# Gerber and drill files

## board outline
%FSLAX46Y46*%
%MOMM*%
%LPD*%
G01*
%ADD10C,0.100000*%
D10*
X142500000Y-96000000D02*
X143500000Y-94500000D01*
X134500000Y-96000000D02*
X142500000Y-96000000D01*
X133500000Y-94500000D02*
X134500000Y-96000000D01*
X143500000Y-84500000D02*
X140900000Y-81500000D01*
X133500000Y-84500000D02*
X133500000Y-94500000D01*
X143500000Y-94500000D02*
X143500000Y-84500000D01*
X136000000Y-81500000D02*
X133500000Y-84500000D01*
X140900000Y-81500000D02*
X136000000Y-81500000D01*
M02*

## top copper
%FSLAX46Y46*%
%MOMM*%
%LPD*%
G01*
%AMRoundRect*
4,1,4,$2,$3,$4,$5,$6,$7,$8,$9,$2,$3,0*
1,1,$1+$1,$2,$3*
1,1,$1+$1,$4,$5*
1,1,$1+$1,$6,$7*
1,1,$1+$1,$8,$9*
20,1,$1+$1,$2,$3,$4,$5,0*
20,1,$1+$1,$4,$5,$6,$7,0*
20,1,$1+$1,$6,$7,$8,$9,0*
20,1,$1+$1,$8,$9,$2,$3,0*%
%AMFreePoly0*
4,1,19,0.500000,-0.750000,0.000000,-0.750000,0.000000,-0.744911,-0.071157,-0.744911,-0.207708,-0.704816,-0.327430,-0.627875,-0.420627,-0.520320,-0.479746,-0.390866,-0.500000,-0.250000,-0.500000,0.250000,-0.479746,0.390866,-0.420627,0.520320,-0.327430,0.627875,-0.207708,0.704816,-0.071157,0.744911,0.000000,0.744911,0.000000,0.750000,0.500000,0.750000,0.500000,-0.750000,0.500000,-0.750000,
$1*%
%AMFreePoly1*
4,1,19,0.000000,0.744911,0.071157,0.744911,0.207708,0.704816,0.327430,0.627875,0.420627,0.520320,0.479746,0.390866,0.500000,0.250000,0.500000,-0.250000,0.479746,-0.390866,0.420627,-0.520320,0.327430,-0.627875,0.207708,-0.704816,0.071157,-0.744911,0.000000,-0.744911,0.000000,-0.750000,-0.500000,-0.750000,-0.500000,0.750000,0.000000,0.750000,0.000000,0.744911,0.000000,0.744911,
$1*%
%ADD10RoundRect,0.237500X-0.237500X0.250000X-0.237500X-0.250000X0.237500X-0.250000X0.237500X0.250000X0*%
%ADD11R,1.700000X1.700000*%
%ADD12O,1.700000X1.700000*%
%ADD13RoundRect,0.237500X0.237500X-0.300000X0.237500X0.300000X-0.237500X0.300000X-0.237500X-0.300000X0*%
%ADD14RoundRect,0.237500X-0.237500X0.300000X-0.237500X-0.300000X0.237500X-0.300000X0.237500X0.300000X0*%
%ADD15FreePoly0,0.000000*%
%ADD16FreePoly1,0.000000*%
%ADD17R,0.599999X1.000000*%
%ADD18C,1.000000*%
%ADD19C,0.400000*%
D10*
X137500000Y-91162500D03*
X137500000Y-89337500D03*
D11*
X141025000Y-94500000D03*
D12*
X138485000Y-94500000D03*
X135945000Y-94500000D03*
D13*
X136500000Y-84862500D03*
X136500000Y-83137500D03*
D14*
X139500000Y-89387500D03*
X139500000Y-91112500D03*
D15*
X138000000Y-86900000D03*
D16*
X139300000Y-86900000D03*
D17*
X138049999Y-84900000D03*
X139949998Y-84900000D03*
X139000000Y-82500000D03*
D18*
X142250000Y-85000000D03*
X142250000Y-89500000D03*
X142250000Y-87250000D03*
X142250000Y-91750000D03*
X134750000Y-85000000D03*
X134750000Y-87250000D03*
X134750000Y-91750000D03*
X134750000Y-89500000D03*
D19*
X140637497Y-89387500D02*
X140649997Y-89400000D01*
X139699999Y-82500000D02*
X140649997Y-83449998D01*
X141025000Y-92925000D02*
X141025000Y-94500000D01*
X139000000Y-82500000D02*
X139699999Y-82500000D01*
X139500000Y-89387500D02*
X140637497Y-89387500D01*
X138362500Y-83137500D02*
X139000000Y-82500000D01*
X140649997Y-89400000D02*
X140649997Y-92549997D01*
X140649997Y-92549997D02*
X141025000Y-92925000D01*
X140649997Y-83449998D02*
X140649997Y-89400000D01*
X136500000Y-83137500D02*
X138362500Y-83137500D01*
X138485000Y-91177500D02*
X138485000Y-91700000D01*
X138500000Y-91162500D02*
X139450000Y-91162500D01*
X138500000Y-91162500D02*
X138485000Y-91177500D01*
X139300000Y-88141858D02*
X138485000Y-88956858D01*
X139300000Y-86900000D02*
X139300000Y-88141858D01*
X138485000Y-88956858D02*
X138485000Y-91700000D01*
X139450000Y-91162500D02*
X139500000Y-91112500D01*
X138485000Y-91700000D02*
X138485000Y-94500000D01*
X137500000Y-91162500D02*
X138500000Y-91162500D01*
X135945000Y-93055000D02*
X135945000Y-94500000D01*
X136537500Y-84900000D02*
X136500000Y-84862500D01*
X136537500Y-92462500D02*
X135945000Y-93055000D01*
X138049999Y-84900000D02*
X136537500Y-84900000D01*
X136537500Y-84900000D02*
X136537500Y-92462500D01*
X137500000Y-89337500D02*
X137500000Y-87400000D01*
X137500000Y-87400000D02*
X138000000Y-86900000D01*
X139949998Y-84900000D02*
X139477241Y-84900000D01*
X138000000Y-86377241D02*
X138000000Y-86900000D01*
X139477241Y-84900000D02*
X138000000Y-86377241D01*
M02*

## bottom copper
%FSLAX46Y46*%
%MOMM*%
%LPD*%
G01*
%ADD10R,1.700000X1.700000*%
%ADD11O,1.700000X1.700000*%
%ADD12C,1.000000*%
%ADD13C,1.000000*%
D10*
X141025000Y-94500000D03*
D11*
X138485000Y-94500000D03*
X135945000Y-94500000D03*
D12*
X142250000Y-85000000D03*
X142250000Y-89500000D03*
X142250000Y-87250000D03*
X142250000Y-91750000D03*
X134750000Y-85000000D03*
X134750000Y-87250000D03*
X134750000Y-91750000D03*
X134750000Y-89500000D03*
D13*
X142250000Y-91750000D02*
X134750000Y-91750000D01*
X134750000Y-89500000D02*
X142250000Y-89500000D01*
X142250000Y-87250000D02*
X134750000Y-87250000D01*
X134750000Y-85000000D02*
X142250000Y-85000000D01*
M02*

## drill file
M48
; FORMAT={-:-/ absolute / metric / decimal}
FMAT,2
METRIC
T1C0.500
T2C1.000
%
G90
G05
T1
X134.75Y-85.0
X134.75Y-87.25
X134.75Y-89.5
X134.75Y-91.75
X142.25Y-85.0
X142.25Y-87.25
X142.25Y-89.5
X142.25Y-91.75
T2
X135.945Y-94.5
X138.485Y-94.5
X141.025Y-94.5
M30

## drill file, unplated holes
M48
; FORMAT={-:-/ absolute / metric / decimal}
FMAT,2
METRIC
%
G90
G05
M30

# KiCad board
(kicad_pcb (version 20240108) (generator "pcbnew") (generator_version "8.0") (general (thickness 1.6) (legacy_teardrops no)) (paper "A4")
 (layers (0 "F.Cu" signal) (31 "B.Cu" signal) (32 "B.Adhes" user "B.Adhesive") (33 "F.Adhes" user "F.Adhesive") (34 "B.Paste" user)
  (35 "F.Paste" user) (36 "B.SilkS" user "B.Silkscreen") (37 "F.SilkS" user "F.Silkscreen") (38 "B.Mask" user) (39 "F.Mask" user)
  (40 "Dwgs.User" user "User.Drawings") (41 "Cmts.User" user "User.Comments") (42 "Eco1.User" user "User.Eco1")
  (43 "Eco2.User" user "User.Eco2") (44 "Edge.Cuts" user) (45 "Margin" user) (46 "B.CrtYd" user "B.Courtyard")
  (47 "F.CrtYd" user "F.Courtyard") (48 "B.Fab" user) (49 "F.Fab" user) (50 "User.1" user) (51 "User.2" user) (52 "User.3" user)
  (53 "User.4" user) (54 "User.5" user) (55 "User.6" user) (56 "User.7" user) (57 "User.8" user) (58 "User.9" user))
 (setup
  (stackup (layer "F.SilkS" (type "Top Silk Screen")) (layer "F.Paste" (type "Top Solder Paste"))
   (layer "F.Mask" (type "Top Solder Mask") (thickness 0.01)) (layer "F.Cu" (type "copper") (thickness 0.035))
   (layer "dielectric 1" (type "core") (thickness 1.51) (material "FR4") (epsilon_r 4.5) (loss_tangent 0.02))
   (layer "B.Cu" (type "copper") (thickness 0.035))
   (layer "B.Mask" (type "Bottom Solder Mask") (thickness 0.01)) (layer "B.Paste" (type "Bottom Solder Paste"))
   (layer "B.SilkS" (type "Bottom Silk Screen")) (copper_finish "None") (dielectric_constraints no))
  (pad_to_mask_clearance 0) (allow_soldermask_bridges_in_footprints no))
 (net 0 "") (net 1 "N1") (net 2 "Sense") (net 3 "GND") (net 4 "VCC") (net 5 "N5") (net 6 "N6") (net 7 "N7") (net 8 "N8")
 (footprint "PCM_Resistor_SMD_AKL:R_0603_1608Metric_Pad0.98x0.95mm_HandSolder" (layer "F.Cu") (at 137.5 90.25 -90)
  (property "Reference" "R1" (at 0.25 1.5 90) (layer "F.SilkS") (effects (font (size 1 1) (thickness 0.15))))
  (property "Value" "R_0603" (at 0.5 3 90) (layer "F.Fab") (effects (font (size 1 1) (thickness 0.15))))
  (pad "1" smd roundrect (at -0.9125 0 270) (size 0.975 0.95) (layers "F.Cu" "F.Paste" "F.Mask") (roundrect_rratio 0.25) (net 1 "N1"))
  (pad "2" smd roundrect (at 0.9125 0 270) (size 0.975 0.95) (layers "F.Cu" "F.Paste" "F.Mask") (roundrect_rratio 0.25) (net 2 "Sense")))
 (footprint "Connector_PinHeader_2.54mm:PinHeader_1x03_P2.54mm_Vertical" (layer "F.Cu") (at 141.025 94.5 -90)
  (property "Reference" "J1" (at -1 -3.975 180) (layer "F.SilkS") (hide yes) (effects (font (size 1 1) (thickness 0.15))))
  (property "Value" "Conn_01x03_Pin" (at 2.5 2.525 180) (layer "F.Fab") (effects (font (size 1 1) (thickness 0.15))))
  (pad "1" thru_hole rect (at 0 0 270) (size 1.7 1.7) (drill 1) (layers "*.Cu" "*.Mask") (remove_unused_layers no) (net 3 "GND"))
  (pad "2" thru_hole oval (at 0 2.54 270) (size 1.7 1.7) (drill 1) (layers "*.Cu" "*.Mask") (remove_unused_layers no) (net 2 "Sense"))
  (pad "3" thru_hole oval (at 0 5.08 270) (size 1.7 1.7) (drill 1) (layers "*.Cu" "*.Mask") (remove_unused_layers no) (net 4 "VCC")))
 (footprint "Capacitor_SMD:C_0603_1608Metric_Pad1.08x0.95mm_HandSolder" (layer "F.Cu") (at 136.5 84 90)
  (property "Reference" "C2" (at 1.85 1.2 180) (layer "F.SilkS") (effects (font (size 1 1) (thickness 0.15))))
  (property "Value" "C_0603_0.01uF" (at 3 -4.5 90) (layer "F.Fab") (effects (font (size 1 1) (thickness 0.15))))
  (pad "1" smd roundrect (at -0.8625 0 90) (size 1.075 0.95) (layers "F.Cu" "F.Paste" "F.Mask") (roundrect_rratio 0.25) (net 4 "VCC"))
  (pad "2" smd roundrect (at 0.8625 0 90) (size 1.075 0.95) (layers "F.Cu" "F.Paste" "F.Mask") (roundrect_rratio 0.25) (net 3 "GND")))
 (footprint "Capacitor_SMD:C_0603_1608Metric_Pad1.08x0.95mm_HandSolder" (layer "F.Cu") (at 139.5 90.25 -90)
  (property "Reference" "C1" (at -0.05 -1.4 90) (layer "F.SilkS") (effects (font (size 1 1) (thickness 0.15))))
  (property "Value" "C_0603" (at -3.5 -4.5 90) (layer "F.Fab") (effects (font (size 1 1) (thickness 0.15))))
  (pad "1" smd roundrect (at -0.8625 0 270) (size 1.075 0.95) (layers "F.Cu" "F.Paste" "F.Mask") (roundrect_rratio 0.25) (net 3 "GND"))
  (pad "2" smd roundrect (at 0.8625 0 270) (size 1.075 0.95) (layers "F.Cu" "F.Paste" "F.Mask") (roundrect_rratio 0.25) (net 2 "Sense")))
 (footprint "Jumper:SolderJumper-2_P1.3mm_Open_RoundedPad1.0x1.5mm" (layer "F.Cu") (at 138.65 86.9)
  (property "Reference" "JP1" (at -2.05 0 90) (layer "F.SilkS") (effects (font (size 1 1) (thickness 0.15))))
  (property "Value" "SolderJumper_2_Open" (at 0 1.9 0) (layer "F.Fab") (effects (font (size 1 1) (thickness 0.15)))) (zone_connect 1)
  (pad "1" smd custom (at -0.65 0) (size 1 0.5) (layers "F.Cu" "F.Mask") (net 1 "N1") (zone_connect 2) (thermal_bridge_angle 45)
   (options (clearance outline) (anchor rect)) (primitives))
  (pad "2" smd custom (at 0.65 0) (size 1 0.5) (layers "F.Cu" "F.Mask") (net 2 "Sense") (zone_connect 2) (thermal_bridge_angle 45)
   (options (clearance outline) (anchor rect)) (primitives)))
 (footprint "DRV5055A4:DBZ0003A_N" (layer "F.Cu") (at 139 83.7 90)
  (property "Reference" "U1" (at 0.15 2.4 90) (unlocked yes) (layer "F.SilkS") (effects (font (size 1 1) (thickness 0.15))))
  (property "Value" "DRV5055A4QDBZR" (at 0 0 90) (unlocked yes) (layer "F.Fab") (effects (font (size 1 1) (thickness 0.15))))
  (pad "1" smd rect (at -1.2 -0.950001 180) (size 0.599999 1) (layers "F.Cu" "F.Paste" "F.Mask") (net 4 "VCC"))
  (pad "2" smd rect (at -1.2 0.949998 180) (size 0.599999 1) (layers "F.Cu" "F.Paste" "F.Mask") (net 1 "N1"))
  (pad "3" smd rect (at 1.2 0 180) (size 0.599999 1) (layers "F.Cu" "F.Paste" "F.Mask") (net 3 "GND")))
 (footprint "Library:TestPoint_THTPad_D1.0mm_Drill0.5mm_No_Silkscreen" (layer "B.Cu") (at 142.25 85 90)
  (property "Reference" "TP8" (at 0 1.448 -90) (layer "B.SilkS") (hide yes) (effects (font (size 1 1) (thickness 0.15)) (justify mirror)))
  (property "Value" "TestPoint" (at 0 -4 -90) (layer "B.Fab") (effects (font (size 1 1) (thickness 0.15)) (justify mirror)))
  (pad "1" thru_hole circle (at 0 0 90) (size 1 1) (drill 0.5) (layers "*.Cu" "*.Mask") (remove_unused_layers no) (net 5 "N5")))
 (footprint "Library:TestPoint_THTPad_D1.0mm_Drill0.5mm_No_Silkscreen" (layer "B.Cu") (at 142.25 89.5 90)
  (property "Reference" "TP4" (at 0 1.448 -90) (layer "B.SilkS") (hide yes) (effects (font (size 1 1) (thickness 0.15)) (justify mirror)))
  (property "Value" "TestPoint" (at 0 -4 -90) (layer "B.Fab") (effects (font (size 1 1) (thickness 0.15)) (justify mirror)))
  (pad "1" thru_hole circle (at 0 0 90) (size 1 1) (drill 0.5) (layers "*.Cu" "*.Mask") (remove_unused_layers no) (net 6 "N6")))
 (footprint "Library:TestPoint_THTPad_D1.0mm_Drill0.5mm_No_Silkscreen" (layer "B.Cu") (at 142.25 87.25 90)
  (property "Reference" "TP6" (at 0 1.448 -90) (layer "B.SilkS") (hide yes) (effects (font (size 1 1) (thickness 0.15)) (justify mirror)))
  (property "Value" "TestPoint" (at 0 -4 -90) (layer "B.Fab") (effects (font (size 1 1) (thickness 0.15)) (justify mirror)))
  (pad "1" thru_hole circle (at 0 0 90) (size 1 1) (drill 0.5) (layers "*.Cu" "*.Mask") (remove_unused_layers no) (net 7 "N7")))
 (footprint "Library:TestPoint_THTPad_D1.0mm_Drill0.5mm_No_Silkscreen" (layer "B.Cu") (at 142.25 91.75 90)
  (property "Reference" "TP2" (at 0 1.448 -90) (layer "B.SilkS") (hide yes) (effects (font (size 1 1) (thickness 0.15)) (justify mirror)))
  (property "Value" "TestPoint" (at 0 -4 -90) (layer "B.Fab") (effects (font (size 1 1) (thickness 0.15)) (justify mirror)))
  (pad "1" thru_hole circle (at 0 0 90) (size 1 1) (drill 0.5) (layers "*.Cu" "*.Mask") (remove_unused_layers no) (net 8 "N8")))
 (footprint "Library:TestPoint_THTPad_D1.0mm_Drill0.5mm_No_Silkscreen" (layer "B.Cu") (at 134.75 85 90)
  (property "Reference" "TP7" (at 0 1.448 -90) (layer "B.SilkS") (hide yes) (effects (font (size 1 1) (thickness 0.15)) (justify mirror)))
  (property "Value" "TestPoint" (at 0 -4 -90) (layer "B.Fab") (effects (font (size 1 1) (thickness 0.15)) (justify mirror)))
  (pad "1" thru_hole circle (at 0 0 90) (size 1 1) (drill 0.5) (layers "*.Cu" "*.Mask") (remove_unused_layers no) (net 5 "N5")))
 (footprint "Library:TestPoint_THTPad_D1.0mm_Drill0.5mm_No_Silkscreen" (layer "B.Cu") (at 134.75 87.25 90)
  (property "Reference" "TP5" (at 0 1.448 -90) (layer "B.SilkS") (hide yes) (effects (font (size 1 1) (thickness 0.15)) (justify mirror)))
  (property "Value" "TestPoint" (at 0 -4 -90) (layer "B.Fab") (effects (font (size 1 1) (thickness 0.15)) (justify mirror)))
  (pad "1" thru_hole circle (at 0 0 90) (size 1 1) (drill 0.5) (layers "*.Cu" "*.Mask") (remove_unused_layers no) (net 7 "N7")))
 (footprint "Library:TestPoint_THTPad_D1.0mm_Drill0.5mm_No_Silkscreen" (layer "B.Cu") (at 134.75 91.75 90)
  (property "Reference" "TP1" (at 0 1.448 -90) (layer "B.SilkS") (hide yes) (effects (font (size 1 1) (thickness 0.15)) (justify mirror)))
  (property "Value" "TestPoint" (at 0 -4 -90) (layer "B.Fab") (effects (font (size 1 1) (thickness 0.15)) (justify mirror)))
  (pad "1" thru_hole circle (at 0 0 90) (size 1 1) (drill 0.5) (layers "*.Cu" "*.Mask") (remove_unused_layers no) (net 8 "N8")))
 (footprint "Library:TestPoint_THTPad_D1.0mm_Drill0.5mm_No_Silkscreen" (layer "B.Cu") (at 134.75 89.5 90)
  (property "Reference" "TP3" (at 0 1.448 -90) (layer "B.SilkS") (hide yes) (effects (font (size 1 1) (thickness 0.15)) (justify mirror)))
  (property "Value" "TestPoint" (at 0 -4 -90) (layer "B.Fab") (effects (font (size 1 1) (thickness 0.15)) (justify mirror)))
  (pad "1" thru_hole circle (at 0 0 90) (size 1 1) (drill 0.5) (layers "*.Cu" "*.Mask") (remove_unused_layers no) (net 6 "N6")))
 (gr_line (start 142.5 96) (end 143.5 94.5) (stroke (width 0.1) (type default)) (layer "Edge.Cuts"))
 (gr_line (start 134.5 96) (end 142.5 96) (stroke (width 0.1) (type default)) (layer "Edge.Cuts"))
 (gr_line (start 133.5 94.5) (end 134.5 96) (stroke (width 0.1) (type default)) (layer "Edge.Cuts"))
 (gr_line (start 143.5 84.5) (end 140.9 81.5) (stroke (width 0.1) (type default)) (layer "Edge.Cuts"))
 (gr_line (start 133.5 84.5) (end 133.5 94.5) (stroke (width 0.1) (type default)) (layer "Edge.Cuts"))
 (gr_line (start 143.5 94.5) (end 143.5 84.5) (stroke (width 0.1) (type default)) (layer "Edge.Cuts"))
 (gr_line (start 136 81.5) (end 133.5 84.5) (stroke (width 0.1) (type default)) (layer "Edge.Cuts"))
 (gr_line (start 140.9 81.5) (end 136 81.5) (stroke (width 0.1) (type default)) (layer "Edge.Cuts"))
 (segment (start 140.637497 89.3875) (end 140.649997 89.4) (width 0.4) (layer "F.Cu") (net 3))
 (segment (start 139.699999 82.5) (end 140.649997 83.449998) (width 0.4) (layer "F.Cu") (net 3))
 (segment (start 141.025 92.925) (end 141.025 94.5) (width 0.4) (layer "F.Cu") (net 3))
 (segment (start 139 82.5) (end 139.699999 82.5) (width 0.4) (layer "F.Cu") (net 3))
 (segment (start 139.5 89.3875) (end 140.637497 89.3875) (width 0.4) (layer "F.Cu") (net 3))
 (segment (start 138.3625 83.1375) (end 139 82.5) (width 0.4) (layer "F.Cu") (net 3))
 (segment (start 140.649997 89.4) (end 140.649997 92.549997) (width 0.4) (layer "F.Cu") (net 3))
 (segment (start 140.649997 92.549997) (end 141.025 92.925) (width 0.4) (layer "F.Cu") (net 3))
 (segment (start 140.649997 83.449998) (end 140.649997 89.4) (width 0.4) (layer "F.Cu") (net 3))
 (segment (start 136.5 83.1375) (end 138.3625 83.1375) (width 0.4) (layer "F.Cu") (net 3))
 (segment (start 138.485 91.1775) (end 138.485 91.7) (width 0.4) (layer "F.Cu") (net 2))
 (segment (start 138.5 91.1625) (end 139.45 91.1625) (width 0.4) (layer "F.Cu") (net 2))
 (segment (start 138.5 91.1625) (end 138.485 91.1775) (width 0.4) (layer "F.Cu") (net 2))
 (segment (start 139.3 88.141858) (end 138.485 88.956858) (width 0.4) (layer "F.Cu") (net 2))
 (segment (start 139.3 86.9) (end 139.3 88.141858) (width 0.4) (layer "F.Cu") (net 2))
 (segment (start 138.485 88.956858) (end 138.485 91.7) (width 0.4) (layer "F.Cu") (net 2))
 (segment (start 139.45 91.1625) (end 139.5 91.1125) (width 0.4) (layer "F.Cu") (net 2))
 (segment (start 138.485 91.7) (end 138.485 94.5) (width 0.4) (layer "F.Cu") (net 2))
 (segment (start 137.5 91.1625) (end 138.5 91.1625) (width 0.4) (layer "F.Cu") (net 2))
 (segment (start 135.945 93.055) (end 135.945 94.5) (width 0.4) (layer "F.Cu") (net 4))
 (segment (start 136.5375 84.9) (end 136.5 84.8625) (width 0.4) (layer "F.Cu") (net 4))
 (segment (start 136.5375 92.4625) (end 135.945 93.055) (width 0.4) (layer "F.Cu") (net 4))
 (segment (start 138.049999 84.9) (end 136.5375 84.9) (width 0.4) (layer "F.Cu") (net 4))
 (segment (start 136.5375 84.9) (end 136.5375 92.4625) (width 0.4) (layer "F.Cu") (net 4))
 (segment (start 137.5 89.3375) (end 137.5 87.4) (width 0.4) (layer "F.Cu") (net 1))
 (segment (start 137.5 87.4) (end 138 86.9) (width 0.4) (layer "F.Cu") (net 1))
 (segment (start 139.949998 84.9) (end 139.477241 84.9) (width 0.4) (layer "F.Cu") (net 1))
 (segment (start 138 86.377241) (end 138 86.9) (width 0.4) (layer "F.Cu") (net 1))
 (segment (start 139.477241 84.9) (end 138 86.377241) (width 0.4) (layer "F.Cu") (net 1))
 (segment (start 142.25 91.75) (end 134.75 91.75) (width 1) (layer "B.Cu") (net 8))
 (segment (start 134.75 89.5) (end 142.25 89.5) (width 1) (layer "B.Cu") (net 6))
 (segment (start 142.25 87.25) (end 134.75 87.25) (width 1) (layer "B.Cu") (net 7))
 (segment (start 134.75 85) (end 142.25 85) (width 1) (layer "B.Cu") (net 5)))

